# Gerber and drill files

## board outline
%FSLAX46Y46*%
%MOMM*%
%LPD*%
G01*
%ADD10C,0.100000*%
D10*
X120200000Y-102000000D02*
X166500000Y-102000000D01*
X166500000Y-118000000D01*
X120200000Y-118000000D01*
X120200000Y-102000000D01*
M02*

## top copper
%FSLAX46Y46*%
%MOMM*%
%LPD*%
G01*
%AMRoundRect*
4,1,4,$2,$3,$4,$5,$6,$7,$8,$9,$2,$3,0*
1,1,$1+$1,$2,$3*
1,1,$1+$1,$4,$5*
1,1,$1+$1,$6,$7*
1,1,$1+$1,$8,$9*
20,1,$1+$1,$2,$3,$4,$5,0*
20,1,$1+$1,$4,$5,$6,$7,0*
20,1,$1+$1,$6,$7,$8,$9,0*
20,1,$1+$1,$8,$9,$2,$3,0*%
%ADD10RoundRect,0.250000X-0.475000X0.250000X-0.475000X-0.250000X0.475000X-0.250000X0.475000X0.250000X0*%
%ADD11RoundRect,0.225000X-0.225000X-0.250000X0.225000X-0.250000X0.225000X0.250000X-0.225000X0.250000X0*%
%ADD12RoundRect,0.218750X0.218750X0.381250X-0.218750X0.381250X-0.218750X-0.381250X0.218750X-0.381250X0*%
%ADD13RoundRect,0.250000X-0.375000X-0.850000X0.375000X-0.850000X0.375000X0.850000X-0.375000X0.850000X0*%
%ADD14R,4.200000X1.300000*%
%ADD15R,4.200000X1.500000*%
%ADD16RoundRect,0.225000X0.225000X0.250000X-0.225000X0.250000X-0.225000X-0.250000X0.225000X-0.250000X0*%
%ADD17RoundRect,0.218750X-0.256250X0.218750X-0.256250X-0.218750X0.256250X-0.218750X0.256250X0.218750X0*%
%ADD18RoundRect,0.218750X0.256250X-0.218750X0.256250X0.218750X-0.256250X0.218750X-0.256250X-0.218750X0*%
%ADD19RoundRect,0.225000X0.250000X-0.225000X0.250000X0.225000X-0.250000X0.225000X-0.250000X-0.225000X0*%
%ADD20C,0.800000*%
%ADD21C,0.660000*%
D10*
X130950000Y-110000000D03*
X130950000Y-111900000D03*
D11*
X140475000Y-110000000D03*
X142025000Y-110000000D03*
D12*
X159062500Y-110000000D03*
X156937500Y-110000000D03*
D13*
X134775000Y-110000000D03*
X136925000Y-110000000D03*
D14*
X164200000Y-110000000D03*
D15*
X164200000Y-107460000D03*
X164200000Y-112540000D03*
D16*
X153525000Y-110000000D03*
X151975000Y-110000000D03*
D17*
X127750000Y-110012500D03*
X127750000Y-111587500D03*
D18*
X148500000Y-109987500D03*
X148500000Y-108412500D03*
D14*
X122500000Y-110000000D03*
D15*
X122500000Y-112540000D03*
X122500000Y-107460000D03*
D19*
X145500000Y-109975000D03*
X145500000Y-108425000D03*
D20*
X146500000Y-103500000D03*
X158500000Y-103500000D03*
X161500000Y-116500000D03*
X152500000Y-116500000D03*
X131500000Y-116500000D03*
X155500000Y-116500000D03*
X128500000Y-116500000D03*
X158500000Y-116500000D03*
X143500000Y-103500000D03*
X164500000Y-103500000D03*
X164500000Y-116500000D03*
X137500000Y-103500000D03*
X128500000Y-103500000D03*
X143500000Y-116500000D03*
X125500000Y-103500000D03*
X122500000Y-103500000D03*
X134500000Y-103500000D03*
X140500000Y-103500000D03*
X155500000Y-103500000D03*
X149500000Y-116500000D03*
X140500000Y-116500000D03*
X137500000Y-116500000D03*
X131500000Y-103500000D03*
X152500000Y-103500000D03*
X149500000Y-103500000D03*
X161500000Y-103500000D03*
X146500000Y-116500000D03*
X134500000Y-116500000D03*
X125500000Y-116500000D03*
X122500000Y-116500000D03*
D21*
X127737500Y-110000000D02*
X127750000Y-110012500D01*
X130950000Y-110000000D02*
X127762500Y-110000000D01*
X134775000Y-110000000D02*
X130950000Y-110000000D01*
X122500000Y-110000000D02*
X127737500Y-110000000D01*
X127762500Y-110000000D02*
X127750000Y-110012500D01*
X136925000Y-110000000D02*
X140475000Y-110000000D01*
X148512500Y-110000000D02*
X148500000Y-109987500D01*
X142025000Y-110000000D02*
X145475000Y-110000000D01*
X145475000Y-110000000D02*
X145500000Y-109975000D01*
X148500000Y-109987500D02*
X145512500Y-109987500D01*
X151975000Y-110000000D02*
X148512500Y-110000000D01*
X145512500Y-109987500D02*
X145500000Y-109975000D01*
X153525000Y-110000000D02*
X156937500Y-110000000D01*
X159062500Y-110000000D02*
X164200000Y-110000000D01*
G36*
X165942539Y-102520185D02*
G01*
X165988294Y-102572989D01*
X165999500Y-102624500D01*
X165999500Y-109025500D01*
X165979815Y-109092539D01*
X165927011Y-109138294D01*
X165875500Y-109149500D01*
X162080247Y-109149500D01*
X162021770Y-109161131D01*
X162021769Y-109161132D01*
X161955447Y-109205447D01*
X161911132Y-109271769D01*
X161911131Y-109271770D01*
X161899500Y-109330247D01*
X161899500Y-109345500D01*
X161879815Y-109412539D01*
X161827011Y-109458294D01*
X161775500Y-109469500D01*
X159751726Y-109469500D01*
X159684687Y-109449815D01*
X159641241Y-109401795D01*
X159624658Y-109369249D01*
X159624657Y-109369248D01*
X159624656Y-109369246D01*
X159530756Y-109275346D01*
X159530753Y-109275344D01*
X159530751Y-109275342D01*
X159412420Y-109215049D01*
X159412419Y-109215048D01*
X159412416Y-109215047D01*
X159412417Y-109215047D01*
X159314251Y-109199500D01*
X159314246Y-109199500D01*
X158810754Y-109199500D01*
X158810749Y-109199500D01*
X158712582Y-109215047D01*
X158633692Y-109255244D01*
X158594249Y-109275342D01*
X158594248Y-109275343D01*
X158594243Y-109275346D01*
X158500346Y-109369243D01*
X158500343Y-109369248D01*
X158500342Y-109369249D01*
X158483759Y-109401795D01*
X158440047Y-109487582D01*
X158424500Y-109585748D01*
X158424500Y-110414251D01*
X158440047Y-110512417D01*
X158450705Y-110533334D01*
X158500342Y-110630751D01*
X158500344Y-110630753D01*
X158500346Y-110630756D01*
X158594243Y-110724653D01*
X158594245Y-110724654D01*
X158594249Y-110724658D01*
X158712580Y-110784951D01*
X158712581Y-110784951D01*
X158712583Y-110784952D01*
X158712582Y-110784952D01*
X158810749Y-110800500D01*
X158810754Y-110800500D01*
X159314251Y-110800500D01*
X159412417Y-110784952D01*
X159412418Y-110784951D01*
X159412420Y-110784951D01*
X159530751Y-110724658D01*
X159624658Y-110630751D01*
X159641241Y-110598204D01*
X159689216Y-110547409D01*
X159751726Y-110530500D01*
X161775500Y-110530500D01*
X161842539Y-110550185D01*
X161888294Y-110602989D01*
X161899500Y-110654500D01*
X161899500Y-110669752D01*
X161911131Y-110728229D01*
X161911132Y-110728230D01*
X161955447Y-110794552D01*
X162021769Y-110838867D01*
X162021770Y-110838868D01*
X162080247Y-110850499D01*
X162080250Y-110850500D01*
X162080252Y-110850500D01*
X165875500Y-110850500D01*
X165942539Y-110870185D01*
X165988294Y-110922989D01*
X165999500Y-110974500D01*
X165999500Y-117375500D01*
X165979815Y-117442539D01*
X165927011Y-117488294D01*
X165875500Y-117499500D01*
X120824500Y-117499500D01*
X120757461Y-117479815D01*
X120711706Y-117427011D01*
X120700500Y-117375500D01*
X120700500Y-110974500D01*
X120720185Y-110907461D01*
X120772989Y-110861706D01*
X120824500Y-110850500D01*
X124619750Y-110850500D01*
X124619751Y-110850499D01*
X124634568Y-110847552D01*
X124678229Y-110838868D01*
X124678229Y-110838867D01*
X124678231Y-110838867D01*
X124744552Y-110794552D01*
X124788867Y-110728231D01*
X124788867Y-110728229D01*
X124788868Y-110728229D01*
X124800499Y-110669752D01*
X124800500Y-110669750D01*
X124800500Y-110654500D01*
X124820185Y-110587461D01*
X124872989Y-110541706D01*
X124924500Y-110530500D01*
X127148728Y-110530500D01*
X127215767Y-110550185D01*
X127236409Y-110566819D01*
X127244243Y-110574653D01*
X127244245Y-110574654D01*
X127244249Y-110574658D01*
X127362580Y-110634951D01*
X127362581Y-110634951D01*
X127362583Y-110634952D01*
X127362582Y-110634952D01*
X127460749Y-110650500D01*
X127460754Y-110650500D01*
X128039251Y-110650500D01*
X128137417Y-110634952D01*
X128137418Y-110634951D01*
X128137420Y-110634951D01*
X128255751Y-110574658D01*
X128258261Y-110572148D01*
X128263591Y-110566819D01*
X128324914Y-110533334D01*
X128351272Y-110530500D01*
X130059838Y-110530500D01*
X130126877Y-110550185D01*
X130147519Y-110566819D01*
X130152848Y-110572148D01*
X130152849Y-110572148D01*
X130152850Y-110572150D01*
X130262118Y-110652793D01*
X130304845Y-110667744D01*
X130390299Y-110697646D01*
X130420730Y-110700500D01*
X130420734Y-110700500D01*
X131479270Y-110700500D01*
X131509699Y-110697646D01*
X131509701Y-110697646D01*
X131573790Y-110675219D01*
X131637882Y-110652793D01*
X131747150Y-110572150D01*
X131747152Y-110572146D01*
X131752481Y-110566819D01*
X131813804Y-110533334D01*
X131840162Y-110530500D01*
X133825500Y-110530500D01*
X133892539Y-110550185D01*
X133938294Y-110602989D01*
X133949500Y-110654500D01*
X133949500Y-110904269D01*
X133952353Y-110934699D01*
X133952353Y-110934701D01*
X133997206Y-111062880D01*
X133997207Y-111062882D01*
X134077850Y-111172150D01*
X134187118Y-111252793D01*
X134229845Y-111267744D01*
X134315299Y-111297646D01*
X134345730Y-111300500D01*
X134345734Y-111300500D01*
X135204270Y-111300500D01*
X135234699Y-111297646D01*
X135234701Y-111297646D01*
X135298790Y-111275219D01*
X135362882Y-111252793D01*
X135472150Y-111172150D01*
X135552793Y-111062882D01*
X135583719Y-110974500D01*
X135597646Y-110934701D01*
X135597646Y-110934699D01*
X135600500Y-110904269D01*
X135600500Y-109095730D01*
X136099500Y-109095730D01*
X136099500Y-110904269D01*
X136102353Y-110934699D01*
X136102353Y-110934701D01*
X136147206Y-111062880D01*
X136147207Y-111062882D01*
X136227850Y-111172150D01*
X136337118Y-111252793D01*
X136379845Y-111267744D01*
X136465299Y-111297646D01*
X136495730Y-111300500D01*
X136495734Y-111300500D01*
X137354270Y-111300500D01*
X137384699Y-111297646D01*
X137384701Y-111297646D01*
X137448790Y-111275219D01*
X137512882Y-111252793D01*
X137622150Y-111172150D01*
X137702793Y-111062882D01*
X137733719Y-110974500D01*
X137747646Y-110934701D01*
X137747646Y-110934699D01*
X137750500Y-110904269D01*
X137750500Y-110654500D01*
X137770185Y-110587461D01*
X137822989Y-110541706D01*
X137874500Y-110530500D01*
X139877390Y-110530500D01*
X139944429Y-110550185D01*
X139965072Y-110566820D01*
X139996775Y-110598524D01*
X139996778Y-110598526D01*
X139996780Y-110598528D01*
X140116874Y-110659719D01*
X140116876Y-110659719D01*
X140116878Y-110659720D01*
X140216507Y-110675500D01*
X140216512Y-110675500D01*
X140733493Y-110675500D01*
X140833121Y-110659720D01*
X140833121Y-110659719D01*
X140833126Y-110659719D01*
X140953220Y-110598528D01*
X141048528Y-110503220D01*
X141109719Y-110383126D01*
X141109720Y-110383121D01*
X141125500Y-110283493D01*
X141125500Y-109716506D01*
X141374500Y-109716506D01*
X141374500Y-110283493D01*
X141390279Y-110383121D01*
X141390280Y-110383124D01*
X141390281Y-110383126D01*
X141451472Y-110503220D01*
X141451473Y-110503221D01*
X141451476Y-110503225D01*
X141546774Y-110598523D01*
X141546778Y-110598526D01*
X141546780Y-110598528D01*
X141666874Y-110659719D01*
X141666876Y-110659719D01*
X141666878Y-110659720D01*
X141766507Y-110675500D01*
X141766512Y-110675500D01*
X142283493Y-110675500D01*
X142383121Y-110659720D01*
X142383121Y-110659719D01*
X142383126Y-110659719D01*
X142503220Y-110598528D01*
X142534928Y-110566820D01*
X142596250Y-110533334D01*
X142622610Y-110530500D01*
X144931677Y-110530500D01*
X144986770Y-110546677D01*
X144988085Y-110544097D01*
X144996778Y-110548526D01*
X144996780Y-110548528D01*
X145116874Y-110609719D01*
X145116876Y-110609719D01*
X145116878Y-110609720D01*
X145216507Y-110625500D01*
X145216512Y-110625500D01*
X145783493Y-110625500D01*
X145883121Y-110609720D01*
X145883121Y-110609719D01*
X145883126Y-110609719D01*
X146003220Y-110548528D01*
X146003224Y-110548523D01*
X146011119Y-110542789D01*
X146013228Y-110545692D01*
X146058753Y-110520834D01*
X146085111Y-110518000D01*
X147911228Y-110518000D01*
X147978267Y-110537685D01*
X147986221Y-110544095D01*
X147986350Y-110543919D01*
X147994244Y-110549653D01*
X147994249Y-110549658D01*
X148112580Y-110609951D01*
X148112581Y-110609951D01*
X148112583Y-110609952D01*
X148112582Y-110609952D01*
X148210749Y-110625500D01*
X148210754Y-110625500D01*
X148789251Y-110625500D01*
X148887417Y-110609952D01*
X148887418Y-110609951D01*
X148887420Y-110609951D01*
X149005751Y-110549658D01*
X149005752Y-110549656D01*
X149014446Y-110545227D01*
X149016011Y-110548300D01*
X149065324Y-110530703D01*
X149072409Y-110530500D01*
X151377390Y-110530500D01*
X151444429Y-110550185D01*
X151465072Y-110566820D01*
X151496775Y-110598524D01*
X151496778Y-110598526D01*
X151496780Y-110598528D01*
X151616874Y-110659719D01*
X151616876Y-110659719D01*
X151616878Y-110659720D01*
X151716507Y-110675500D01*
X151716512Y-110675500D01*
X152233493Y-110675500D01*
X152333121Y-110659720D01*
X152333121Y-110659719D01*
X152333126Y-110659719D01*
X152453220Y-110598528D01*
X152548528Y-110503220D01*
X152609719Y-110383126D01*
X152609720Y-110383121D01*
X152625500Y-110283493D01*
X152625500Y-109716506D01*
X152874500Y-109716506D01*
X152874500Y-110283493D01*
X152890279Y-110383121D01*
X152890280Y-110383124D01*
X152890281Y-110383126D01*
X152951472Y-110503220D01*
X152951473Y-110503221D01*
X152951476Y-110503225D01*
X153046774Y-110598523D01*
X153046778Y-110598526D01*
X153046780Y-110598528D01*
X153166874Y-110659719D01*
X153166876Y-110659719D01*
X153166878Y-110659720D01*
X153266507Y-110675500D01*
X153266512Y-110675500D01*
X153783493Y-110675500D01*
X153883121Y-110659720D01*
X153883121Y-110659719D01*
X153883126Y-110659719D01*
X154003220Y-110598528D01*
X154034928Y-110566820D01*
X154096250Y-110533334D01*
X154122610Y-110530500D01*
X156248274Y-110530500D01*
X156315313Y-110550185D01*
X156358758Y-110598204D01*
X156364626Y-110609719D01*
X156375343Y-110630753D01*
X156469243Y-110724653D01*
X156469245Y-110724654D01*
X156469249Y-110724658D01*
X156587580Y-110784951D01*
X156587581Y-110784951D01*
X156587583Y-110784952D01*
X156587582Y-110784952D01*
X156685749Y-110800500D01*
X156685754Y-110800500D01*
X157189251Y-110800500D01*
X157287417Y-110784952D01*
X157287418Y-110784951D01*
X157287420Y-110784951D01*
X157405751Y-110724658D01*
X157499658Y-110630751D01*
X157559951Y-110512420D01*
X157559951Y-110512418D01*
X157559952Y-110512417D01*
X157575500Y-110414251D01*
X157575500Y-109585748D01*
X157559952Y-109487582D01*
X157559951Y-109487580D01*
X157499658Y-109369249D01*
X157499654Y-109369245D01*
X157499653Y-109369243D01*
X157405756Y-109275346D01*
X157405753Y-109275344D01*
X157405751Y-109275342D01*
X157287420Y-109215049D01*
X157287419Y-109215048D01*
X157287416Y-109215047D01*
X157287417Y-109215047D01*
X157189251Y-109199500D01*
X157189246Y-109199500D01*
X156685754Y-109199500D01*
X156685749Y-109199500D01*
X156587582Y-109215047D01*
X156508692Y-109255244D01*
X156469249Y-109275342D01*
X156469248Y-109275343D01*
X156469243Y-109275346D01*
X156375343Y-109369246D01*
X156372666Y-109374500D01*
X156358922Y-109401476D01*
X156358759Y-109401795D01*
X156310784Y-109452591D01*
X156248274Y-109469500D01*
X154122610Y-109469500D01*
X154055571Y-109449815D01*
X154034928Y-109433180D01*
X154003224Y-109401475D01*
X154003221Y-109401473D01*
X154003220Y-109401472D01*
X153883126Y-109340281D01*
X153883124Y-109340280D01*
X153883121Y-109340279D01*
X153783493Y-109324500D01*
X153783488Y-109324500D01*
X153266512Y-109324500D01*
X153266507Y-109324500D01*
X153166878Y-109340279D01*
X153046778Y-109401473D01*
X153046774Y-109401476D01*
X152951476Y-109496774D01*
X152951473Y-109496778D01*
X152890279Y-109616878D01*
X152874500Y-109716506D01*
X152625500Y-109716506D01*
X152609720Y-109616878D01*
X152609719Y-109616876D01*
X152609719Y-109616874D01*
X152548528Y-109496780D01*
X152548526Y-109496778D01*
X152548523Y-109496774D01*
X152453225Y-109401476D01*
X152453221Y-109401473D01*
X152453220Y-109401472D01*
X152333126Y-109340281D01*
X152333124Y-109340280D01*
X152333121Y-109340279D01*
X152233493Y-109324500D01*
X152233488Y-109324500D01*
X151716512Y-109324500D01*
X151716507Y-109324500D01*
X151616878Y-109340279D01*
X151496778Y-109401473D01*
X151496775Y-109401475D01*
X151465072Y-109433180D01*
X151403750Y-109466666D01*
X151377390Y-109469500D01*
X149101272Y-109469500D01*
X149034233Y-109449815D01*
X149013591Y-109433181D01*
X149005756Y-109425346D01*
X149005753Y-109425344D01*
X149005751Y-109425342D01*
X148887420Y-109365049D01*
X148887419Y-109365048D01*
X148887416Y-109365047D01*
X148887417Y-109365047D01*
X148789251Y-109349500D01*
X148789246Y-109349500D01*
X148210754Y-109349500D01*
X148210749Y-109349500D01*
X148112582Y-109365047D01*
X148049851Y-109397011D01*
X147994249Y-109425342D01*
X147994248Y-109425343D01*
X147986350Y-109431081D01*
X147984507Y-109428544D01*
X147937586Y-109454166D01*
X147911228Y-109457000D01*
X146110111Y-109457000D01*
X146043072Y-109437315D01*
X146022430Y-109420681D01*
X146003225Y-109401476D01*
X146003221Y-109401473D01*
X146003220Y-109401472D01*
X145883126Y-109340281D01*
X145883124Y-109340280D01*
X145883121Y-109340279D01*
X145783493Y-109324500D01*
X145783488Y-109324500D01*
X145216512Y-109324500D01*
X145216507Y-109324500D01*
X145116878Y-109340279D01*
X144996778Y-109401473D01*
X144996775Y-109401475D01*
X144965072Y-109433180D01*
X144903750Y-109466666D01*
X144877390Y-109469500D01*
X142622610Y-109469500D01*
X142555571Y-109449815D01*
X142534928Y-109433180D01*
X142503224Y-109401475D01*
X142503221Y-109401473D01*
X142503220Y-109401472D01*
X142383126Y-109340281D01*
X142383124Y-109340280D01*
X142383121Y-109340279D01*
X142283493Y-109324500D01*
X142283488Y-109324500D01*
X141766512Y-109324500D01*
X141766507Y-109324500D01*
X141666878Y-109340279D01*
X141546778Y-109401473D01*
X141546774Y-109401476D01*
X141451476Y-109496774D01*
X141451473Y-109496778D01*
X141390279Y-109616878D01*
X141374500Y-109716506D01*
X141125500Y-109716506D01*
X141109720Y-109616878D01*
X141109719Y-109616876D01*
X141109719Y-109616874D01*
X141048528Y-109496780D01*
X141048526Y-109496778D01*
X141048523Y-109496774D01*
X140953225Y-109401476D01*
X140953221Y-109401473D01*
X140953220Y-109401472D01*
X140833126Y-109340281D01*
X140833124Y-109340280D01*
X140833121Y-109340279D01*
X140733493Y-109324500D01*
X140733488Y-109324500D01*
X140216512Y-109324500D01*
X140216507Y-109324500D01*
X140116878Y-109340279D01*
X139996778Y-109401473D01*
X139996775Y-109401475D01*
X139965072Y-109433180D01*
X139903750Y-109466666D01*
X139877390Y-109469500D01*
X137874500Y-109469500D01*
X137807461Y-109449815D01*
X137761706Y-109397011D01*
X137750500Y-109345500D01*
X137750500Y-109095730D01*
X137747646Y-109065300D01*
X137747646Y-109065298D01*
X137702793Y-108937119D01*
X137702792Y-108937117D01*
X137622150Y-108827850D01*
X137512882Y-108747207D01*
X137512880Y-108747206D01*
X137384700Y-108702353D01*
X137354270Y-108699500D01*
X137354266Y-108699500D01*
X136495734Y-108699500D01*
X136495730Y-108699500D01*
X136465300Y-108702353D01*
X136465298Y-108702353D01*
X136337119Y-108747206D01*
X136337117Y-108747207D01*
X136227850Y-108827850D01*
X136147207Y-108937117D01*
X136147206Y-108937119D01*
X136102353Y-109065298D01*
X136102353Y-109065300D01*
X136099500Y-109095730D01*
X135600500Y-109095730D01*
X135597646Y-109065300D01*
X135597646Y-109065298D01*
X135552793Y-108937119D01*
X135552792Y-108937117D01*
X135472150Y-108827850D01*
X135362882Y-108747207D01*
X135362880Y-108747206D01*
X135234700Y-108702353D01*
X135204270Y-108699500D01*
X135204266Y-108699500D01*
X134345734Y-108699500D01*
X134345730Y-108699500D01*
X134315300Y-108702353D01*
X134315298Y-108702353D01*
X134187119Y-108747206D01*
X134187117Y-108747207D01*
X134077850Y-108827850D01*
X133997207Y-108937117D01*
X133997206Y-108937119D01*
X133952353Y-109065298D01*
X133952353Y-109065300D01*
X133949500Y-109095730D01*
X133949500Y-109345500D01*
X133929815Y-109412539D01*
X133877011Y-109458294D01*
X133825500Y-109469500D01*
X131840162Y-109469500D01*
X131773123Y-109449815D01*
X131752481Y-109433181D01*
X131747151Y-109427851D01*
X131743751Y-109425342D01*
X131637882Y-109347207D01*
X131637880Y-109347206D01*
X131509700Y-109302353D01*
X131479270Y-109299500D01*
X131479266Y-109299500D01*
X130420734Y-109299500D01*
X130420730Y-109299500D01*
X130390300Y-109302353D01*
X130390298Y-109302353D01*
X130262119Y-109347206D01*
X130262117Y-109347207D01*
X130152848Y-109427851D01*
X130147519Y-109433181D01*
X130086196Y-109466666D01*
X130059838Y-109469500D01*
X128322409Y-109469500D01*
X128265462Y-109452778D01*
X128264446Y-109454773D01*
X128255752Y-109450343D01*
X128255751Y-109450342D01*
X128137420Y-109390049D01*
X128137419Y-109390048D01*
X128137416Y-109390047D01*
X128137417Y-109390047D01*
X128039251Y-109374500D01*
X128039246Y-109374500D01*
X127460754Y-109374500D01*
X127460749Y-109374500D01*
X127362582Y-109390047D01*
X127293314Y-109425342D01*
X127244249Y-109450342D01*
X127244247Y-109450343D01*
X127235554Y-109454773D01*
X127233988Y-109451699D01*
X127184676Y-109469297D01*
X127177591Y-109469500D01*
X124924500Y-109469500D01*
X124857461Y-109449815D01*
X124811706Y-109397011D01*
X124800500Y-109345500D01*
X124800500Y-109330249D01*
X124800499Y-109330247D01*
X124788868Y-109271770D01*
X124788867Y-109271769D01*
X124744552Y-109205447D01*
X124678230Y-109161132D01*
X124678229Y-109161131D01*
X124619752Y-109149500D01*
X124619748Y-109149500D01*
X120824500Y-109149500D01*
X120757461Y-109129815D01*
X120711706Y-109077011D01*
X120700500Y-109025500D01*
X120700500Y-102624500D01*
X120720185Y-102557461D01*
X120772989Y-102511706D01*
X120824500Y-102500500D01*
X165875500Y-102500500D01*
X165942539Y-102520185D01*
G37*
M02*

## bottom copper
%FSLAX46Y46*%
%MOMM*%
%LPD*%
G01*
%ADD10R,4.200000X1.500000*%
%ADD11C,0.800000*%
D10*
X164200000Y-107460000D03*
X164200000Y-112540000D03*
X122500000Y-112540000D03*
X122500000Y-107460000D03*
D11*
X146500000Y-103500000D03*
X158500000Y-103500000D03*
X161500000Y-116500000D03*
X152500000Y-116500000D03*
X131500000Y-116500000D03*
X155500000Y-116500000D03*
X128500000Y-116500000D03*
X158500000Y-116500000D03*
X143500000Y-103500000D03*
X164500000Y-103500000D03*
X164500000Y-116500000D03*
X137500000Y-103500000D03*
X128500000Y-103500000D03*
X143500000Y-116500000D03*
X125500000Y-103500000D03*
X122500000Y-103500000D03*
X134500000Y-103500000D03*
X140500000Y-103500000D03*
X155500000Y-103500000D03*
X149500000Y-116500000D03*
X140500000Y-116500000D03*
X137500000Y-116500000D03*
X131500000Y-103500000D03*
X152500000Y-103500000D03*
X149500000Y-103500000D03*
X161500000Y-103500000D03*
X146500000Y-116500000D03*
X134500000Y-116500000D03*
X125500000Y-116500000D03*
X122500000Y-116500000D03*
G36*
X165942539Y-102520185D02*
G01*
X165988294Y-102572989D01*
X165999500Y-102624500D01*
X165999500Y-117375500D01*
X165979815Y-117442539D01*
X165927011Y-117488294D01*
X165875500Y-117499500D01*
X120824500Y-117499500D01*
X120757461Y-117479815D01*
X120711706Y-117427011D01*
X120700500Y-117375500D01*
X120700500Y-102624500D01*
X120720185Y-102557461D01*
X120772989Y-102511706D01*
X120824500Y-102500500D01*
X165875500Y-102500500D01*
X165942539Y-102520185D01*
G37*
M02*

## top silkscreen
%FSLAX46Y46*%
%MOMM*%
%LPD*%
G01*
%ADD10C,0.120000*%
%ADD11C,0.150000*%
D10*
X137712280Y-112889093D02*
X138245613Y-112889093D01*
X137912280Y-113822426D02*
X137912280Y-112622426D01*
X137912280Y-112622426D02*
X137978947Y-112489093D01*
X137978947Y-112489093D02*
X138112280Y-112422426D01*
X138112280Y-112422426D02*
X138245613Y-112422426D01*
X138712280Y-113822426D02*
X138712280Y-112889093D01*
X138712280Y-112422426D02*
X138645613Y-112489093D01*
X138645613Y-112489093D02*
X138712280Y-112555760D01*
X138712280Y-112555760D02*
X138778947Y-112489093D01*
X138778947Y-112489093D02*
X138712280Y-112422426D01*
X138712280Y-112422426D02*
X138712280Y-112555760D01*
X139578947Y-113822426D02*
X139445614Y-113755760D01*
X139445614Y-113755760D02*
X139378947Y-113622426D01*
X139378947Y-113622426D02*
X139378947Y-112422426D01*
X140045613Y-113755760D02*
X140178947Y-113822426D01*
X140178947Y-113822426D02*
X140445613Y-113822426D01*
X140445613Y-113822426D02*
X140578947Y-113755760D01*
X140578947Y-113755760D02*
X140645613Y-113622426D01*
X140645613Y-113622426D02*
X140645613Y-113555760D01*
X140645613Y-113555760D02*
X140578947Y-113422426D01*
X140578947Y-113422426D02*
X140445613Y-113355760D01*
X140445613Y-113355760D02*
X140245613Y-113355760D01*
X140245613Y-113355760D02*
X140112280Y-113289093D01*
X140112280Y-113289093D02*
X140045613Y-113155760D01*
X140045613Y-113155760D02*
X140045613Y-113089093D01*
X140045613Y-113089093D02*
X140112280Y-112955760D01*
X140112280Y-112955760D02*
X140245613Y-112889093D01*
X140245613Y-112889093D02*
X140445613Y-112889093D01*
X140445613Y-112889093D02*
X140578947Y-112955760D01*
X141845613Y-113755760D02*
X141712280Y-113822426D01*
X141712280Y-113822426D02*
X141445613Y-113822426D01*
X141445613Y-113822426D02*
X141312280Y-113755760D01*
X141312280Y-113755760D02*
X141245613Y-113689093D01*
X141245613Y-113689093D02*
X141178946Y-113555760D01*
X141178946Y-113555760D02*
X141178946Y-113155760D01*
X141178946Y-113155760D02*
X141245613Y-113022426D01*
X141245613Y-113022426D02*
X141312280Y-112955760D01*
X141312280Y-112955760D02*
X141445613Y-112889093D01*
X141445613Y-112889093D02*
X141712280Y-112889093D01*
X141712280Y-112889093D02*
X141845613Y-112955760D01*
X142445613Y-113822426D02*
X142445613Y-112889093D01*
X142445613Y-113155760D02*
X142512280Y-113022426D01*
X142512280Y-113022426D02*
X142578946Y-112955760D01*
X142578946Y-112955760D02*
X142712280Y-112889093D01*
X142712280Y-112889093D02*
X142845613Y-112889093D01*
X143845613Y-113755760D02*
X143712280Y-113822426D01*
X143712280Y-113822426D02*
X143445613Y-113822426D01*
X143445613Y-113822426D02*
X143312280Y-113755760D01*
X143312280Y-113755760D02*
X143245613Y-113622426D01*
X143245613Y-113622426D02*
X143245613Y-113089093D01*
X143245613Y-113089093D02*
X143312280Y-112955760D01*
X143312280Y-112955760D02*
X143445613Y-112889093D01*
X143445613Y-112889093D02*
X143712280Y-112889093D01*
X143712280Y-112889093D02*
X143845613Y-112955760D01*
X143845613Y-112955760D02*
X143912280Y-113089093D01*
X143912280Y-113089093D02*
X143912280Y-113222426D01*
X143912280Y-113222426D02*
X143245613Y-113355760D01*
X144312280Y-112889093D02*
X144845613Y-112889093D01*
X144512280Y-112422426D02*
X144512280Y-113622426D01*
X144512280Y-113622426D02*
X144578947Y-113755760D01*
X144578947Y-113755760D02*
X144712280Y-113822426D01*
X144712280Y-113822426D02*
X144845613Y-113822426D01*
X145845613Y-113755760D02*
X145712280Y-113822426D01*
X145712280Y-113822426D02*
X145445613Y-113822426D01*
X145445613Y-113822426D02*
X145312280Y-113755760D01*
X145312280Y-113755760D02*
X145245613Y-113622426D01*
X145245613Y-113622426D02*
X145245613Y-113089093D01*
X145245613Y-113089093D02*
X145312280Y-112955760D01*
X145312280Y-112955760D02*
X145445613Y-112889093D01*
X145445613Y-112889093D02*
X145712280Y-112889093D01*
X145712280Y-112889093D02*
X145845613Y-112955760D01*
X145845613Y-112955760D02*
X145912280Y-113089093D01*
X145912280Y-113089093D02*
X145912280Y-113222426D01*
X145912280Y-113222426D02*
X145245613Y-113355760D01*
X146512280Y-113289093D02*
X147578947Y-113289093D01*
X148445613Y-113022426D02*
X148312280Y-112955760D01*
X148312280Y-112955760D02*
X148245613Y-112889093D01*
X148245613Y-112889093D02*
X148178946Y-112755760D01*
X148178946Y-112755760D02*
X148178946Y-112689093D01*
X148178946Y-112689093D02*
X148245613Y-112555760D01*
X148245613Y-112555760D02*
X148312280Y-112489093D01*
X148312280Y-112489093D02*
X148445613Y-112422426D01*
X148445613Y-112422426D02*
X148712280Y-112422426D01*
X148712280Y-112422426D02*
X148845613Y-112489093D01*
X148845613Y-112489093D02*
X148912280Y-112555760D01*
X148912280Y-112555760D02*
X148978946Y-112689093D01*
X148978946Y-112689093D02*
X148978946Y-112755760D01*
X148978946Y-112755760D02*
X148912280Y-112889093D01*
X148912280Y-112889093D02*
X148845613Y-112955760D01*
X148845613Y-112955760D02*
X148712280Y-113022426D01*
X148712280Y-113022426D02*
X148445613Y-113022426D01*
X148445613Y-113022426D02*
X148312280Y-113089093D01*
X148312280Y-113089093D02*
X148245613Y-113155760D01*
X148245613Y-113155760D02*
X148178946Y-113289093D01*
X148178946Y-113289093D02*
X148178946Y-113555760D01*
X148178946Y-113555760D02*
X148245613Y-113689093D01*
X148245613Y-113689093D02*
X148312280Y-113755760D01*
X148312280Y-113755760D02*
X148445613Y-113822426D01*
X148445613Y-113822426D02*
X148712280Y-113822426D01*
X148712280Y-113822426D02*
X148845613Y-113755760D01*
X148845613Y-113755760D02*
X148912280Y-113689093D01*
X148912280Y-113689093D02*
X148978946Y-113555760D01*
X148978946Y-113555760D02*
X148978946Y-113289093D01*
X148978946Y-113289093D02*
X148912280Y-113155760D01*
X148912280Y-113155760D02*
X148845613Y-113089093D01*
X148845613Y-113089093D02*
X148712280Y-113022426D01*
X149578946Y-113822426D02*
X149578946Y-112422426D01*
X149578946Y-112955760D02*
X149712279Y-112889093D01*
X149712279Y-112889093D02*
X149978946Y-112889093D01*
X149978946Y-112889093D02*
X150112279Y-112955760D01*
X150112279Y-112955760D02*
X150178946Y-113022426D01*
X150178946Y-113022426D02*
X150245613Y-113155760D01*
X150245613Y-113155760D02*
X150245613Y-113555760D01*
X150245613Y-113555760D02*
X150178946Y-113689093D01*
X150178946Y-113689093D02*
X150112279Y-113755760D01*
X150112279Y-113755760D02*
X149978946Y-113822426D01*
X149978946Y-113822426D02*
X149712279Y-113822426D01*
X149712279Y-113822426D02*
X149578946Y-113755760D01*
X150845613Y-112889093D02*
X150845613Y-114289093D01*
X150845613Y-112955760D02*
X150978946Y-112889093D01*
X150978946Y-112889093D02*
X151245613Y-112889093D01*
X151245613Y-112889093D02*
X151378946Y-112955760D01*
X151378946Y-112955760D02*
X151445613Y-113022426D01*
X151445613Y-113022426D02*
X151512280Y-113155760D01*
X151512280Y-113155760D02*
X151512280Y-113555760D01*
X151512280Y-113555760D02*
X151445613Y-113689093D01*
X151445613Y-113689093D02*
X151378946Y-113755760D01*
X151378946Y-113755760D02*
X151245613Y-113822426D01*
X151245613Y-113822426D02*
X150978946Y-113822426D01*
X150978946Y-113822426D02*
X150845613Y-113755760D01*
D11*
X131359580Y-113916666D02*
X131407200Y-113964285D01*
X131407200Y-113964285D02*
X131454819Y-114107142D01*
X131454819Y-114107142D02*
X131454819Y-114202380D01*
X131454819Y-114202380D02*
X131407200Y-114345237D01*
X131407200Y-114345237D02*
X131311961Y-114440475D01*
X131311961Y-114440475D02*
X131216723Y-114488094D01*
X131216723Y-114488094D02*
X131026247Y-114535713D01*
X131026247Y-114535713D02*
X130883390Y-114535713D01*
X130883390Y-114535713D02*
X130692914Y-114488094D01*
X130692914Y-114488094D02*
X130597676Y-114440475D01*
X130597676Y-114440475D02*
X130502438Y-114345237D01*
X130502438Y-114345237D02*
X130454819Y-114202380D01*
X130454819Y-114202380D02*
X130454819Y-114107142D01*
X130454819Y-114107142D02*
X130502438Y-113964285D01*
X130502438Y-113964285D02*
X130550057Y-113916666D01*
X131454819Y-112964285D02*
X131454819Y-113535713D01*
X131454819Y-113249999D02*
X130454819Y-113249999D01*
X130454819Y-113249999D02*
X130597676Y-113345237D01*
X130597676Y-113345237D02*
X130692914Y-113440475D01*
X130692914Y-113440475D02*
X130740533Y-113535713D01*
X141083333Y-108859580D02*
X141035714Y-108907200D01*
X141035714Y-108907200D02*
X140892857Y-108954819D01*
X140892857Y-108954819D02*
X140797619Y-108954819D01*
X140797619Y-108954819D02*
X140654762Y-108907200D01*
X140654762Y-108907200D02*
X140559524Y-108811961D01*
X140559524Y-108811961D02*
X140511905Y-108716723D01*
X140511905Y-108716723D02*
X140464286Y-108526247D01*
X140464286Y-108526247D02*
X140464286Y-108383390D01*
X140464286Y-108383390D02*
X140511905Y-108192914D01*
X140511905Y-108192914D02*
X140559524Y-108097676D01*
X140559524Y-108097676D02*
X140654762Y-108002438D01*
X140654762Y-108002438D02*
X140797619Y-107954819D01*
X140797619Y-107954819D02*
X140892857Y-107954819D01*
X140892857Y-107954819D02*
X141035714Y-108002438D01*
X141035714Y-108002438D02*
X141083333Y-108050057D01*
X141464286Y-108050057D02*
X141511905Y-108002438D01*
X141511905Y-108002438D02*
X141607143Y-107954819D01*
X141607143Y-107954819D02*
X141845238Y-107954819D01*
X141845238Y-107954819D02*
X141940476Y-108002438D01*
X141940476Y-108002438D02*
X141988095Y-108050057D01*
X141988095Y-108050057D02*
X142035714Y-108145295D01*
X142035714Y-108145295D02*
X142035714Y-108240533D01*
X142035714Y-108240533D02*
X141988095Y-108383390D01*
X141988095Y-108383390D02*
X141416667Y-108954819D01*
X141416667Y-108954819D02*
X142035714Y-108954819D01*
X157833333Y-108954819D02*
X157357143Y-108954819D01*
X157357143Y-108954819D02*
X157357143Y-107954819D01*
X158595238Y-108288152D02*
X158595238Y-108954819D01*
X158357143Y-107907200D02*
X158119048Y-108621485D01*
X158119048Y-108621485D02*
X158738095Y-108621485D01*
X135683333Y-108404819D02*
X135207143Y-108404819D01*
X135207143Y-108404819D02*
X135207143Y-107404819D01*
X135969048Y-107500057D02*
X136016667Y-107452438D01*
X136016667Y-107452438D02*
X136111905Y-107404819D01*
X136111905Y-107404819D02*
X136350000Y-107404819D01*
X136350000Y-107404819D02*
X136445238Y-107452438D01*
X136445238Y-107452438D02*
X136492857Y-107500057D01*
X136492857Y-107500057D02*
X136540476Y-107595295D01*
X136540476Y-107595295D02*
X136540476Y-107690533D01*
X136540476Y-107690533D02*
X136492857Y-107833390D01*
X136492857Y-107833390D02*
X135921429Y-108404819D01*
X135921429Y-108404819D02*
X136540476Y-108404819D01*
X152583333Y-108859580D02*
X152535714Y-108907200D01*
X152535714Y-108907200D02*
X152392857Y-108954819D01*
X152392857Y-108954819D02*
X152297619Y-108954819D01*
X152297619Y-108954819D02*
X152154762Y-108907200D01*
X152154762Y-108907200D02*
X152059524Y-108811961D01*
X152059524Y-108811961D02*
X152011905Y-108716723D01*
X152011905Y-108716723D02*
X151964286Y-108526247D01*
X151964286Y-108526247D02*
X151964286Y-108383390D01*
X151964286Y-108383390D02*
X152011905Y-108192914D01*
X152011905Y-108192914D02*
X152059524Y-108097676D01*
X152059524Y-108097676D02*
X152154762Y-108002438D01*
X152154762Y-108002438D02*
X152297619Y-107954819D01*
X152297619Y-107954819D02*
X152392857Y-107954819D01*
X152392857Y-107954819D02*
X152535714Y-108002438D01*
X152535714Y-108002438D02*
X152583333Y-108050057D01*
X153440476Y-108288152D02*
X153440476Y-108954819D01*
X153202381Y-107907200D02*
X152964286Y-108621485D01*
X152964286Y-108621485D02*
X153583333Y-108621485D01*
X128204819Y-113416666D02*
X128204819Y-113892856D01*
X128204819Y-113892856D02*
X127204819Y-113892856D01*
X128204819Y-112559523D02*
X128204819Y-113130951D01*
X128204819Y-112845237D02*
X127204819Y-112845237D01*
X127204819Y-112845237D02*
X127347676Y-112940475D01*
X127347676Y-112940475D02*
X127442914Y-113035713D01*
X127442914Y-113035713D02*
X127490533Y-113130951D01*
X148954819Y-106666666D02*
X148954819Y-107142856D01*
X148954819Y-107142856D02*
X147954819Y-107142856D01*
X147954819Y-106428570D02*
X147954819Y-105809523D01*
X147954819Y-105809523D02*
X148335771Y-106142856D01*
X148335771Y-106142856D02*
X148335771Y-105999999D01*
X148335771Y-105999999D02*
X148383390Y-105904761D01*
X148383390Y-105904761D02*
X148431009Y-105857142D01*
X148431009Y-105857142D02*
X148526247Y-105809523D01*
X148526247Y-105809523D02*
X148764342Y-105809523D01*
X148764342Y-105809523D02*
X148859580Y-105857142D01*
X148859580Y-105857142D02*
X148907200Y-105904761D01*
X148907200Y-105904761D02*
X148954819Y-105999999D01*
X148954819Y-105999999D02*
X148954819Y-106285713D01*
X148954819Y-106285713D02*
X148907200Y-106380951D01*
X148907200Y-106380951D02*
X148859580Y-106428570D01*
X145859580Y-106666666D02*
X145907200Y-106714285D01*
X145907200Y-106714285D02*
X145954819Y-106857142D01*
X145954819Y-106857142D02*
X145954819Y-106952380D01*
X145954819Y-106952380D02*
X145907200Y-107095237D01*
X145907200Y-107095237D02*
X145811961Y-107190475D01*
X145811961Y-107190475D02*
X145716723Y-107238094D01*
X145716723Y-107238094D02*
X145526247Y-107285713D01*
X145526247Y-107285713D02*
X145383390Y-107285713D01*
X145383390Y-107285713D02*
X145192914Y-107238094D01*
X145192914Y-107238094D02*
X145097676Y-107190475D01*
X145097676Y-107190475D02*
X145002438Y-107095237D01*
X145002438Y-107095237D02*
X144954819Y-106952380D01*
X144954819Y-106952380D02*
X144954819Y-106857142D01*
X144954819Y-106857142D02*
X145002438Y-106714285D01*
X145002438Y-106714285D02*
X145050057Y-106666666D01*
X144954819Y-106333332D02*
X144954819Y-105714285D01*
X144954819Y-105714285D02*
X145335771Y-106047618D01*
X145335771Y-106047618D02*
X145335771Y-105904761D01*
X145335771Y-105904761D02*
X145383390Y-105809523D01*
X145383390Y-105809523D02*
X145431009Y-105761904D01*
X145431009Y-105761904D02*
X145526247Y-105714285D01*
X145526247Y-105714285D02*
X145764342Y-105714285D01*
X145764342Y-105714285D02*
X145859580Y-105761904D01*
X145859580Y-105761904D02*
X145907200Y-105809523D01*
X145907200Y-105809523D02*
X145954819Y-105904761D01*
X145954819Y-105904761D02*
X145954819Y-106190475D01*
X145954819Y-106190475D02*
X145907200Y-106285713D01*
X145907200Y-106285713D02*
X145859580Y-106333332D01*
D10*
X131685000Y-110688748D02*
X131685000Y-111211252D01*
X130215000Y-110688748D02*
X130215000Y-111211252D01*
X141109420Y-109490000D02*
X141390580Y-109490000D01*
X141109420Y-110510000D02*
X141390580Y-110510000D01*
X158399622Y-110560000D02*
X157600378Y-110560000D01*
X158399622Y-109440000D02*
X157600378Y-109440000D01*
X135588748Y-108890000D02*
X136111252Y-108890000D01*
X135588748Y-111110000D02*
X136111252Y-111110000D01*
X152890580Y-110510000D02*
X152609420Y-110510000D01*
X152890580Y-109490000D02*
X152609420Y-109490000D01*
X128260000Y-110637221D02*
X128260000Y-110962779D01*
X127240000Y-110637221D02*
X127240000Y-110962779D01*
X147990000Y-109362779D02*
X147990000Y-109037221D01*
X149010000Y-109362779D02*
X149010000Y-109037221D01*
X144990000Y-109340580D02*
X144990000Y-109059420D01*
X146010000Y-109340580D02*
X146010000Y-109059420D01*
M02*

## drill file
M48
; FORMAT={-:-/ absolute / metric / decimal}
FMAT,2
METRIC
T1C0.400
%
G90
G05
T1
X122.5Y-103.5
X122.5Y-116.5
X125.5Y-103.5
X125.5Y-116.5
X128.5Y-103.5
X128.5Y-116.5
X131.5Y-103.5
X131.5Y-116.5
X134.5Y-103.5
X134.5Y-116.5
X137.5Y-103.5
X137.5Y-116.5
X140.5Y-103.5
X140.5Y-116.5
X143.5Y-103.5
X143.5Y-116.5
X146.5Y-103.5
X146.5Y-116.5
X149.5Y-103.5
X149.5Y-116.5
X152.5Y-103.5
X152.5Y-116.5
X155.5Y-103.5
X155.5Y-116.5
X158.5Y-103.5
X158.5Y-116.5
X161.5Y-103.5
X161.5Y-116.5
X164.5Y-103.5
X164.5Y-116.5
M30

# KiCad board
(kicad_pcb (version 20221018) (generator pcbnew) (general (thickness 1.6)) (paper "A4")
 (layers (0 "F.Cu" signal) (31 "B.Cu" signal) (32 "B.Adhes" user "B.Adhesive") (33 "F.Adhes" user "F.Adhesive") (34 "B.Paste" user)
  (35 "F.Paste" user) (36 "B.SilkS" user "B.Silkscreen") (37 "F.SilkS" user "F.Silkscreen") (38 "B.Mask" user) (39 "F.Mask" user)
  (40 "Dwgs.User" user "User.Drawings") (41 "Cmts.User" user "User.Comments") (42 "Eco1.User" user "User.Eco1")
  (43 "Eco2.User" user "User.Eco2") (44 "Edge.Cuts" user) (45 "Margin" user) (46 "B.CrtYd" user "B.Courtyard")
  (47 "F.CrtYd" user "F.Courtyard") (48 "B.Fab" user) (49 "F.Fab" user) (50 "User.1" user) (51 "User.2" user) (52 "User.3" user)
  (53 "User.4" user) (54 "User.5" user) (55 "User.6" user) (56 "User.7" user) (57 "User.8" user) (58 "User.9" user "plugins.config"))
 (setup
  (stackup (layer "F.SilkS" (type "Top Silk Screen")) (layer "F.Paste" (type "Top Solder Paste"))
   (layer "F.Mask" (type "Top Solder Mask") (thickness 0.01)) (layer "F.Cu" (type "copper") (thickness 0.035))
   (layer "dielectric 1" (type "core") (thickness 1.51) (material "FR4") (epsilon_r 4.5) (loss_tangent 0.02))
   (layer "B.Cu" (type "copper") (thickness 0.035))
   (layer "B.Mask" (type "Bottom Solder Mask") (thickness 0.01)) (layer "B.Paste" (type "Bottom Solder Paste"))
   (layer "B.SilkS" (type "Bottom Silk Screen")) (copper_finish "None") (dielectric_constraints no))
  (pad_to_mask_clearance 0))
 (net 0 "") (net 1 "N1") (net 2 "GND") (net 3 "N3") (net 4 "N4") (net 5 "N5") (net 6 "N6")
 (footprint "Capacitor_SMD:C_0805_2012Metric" (layer "F.Cu") (at 130.95 110.95 -90)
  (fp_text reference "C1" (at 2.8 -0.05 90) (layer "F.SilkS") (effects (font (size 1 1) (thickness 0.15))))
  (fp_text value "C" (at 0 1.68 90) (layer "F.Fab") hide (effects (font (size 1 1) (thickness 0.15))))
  (fp_line (start -0.261252 -0.735) (end 0.261252 -0.735) (stroke (width 0.12) (type solid)) (layer "F.SilkS"))
  (fp_line (start -0.261252 0.735) (end 0.261252 0.735) (stroke (width 0.12) (type solid)) (layer "F.SilkS"))
  (pad "1" smd roundrect (at -0.95 0 270) (size 1 1.45) (layers "F.Cu" "F.Paste" "F.Mask") (roundrect_rratio 0.25) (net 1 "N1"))
  (pad "2" smd roundrect (at 0.95 0 270) (size 1 1.45) (layers "F.Cu" "F.Paste" "F.Mask") (roundrect_rratio 0.25) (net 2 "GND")))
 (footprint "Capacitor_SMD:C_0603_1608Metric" (layer "F.Cu") (at 141.25 110)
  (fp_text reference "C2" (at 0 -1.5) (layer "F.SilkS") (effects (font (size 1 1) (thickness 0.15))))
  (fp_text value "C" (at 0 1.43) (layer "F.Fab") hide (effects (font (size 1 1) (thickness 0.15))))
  (fp_line (start -0.14058 -0.51) (end 0.14058 -0.51) (stroke (width 0.12) (type solid)) (layer "F.SilkS"))
  (fp_line (start -0.14058 0.51) (end 0.14058 0.51) (stroke (width 0.12) (type solid)) (layer "F.SilkS"))
  (pad "1" smd roundrect (at -0.775 0) (size 0.9 0.95) (layers "F.Cu" "F.Paste" "F.Mask") (roundrect_rratio 0.25) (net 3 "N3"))
  (pad "2" smd roundrect (at 0.775 0) (size 0.9 0.95) (layers "F.Cu" "F.Paste" "F.Mask") (roundrect_rratio 0.25) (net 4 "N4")))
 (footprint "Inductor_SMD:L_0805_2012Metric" (layer "F.Cu") (at 158 110 180)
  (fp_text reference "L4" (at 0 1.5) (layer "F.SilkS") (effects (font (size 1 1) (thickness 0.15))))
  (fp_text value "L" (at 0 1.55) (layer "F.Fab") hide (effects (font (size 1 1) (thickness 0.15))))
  (fp_line (start -0.399622 -0.56) (end 0.399622 -0.56) (stroke (width 0.12) (type solid)) (layer "F.SilkS"))
  (fp_line (start -0.399622 0.56) (end 0.399622 0.56) (stroke (width 0.12) (type solid)) (layer "F.SilkS"))
  (pad "1" smd roundrect (at -1.0625 0 180) (size 0.875 1.2) (layers "F.Cu" "F.Paste" "F.Mask") (roundrect_rratio 0.25) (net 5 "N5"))
  (pad "2" smd roundrect (at 1.0625 0 180) (size 0.875 1.2) (layers "F.Cu" "F.Paste" "F.Mask") (roundrect_rratio 0.25) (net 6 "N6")))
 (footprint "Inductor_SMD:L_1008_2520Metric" (layer "F.Cu") (at 135.85 110)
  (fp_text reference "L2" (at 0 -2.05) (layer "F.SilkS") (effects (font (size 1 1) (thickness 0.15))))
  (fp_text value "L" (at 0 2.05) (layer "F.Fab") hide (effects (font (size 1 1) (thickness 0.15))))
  (fp_line (start -0.261252 -1.11) (end 0.261252 -1.11) (stroke (width 0.12) (type solid)) (layer "F.SilkS"))
  (fp_line (start -0.261252 1.11) (end 0.261252 1.11) (stroke (width 0.12) (type solid)) (layer "F.SilkS"))
  (pad "1" smd roundrect (at -1.075 0) (size 1.25 2.2) (layers "F.Cu" "F.Paste" "F.Mask") (roundrect_rratio 0.2) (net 1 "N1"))
  (pad "2" smd roundrect (at 1.075 0) (size 1.25 2.2) (layers "F.Cu" "F.Paste" "F.Mask") (roundrect_rratio 0.2) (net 3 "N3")))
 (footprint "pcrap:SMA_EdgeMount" (layer "F.Cu") (at 163.2 110 -90)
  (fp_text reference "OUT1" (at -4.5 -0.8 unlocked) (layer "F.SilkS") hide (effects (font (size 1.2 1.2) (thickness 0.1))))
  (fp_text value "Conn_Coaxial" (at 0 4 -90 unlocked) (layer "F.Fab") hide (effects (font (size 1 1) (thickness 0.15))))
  (pad "1" smd rect (at 0 -1 90) (size 1.3 4.2) (layers "F.Cu" "F.Paste" "F.Mask") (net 5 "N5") (thermal_bridge_angle 45))
  (pad "2" smd rect (at -2.54 -1 90) (size 1.5 4.2) (layers "F.Cu" "F.Paste" "F.Mask") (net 2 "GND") (thermal_bridge_angle 45))
  (pad "2" smd rect (at -2.54 -1 270) (size 1.5 4.2) (layers "B.Cu" "B.Paste" "B.Mask") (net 2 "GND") (thermal_bridge_angle 45))
  (pad "2" smd rect (at 2.54 -1 90) (size 1.5 4.2) (layers "F.Cu" "F.Paste" "F.Mask") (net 2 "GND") (thermal_bridge_angle 45))
  (pad "2" smd rect (at 2.54 -1 90) (size 1.5 4.2) (layers "B.Cu" "B.Paste" "B.Mask") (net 2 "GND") (thermal_bridge_angle 45)))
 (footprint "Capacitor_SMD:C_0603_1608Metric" (layer "F.Cu") (at 152.75 110 180)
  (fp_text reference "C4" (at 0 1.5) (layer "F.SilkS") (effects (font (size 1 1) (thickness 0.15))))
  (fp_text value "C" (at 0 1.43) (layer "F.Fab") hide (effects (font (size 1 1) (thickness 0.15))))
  (fp_line (start -0.14058 -0.51) (end 0.14058 -0.51) (stroke (width 0.12) (type solid)) (layer "F.SilkS"))
  (fp_line (start -0.14058 0.51) (end 0.14058 0.51) (stroke (width 0.12) (type solid)) (layer "F.SilkS"))
  (pad "1" smd roundrect (at -0.775 0 180) (size 0.9 0.95) (layers "F.Cu" "F.Paste" "F.Mask") (roundrect_rratio 0.25) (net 6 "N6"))
  (pad "2" smd roundrect (at 0.775 0 180) (size 0.9 0.95) (layers "F.Cu" "F.Paste" "F.Mask") (roundrect_rratio 0.25) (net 4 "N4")))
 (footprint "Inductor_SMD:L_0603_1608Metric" (layer "F.Cu") (at 127.75 110.8 -90)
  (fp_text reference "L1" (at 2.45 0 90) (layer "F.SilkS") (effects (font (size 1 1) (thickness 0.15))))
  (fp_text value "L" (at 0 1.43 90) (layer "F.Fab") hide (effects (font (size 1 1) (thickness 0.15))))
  (fp_line (start -0.162779 -0.51) (end 0.162779 -0.51) (stroke (width 0.12) (type solid)) (layer "F.SilkS"))
  (fp_line (start -0.162779 0.51) (end 0.162779 0.51) (stroke (width 0.12) (type solid)) (layer "F.SilkS"))
  (pad "1" smd roundrect (at -0.7875 0 270) (size 0.875 0.95) (layers "F.Cu" "F.Paste" "F.Mask") (roundrect_rratio 0.25) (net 1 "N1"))
  (pad "2" smd roundrect (at 0.7875 0 270) (size 0.875 0.95) (layers "F.Cu" "F.Paste" "F.Mask") (roundrect_rratio 0.25) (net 2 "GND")))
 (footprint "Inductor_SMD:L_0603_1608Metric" (layer "F.Cu") (at 148.5 109.2 90)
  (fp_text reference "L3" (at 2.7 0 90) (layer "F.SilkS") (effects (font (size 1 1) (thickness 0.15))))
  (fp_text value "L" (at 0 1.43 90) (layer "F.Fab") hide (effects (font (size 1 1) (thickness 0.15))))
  (fp_line (start -0.162779 -0.51) (end 0.162779 -0.51) (stroke (width 0.12) (type solid)) (layer "F.SilkS"))
  (fp_line (start -0.162779 0.51) (end 0.162779 0.51) (stroke (width 0.12) (type solid)) (layer "F.SilkS"))
  (pad "1" smd roundrect (at -0.7875 0 90) (size 0.875 0.95) (layers "F.Cu" "F.Paste" "F.Mask") (roundrect_rratio 0.25) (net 4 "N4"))
  (pad "2" smd roundrect (at 0.7875 0 90) (size 0.875 0.95) (layers "F.Cu" "F.Paste" "F.Mask") (roundrect_rratio 0.25) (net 2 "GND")))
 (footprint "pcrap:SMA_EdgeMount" (layer "F.Cu") (at 123.5 110 90)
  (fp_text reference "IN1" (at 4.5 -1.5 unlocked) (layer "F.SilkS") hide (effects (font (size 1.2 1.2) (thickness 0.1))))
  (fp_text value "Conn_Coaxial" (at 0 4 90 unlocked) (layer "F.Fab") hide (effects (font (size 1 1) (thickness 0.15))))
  (pad "1" smd rect (at 0 -1 270) (size 1.3 4.2) (layers "F.Cu" "F.Paste" "F.Mask") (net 1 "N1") (thermal_bridge_angle 45))
  (pad "2" smd rect (at -2.54 -1 270) (size 1.5 4.2) (layers "F.Cu" "F.Paste" "F.Mask") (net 2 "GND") (thermal_bridge_angle 45))
  (pad "2" smd rect (at -2.54 -1 90) (size 1.5 4.2) (layers "B.Cu" "B.Paste" "B.Mask") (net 2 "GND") (thermal_bridge_angle 45))
  (pad "2" smd rect (at 2.54 -1 270) (size 1.5 4.2) (layers "F.Cu" "F.Paste" "F.Mask") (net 2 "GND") (thermal_bridge_angle 45))
  (pad "2" smd rect (at 2.54 -1 270) (size 1.5 4.2) (layers "B.Cu" "B.Paste" "B.Mask") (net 2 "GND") (thermal_bridge_angle 45)))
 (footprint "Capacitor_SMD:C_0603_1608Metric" (layer "F.Cu") (at 145.5 109.2 90)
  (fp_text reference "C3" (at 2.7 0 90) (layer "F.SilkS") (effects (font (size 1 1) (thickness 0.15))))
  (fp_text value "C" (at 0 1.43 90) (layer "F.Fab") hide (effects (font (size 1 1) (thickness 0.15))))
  (fp_line (start -0.14058 -0.51) (end 0.14058 -0.51) (stroke (width 0.12) (type solid)) (layer "F.SilkS"))
  (fp_line (start -0.14058 0.51) (end 0.14058 0.51) (stroke (width 0.12) (type solid)) (layer "F.SilkS"))
  (pad "1" smd roundrect (at -0.775 0 90) (size 0.9 0.95) (layers "F.Cu" "F.Paste" "F.Mask") (roundrect_rratio 0.25) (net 4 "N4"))
  (pad "2" smd roundrect (at 0.775 0 90) (size 0.9 0.95) (layers "F.Cu" "F.Paste" "F.Mask") (roundrect_rratio 0.25) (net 2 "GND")))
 (gr_rect (start 120.2 102) (end 166.5 118) (stroke (width 0.1) (type default)) (fill none) (layer "Edge.Cuts"))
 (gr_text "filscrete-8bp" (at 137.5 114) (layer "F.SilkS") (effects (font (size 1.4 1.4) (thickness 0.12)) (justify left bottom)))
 (segment (start 127.7375 110) (end 127.75 110.0125) (width 0.66) (layer "F.Cu") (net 1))
 (segment (start 130.95 110) (end 127.7625 110) (width 0.66) (layer "F.Cu") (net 1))
 (segment (start 134.775 110) (end 130.95 110) (width 0.66) (layer "F.Cu") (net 1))
 (segment (start 122.5 110) (end 127.7375 110) (width 0.66) (layer "F.Cu") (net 1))
 (segment (start 127.7625 110) (end 127.75 110.0125) (width 0.66) (layer "F.Cu") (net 1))
 (via (at 146.5 103.5) (size 0.8) (drill 0.4) (layers "F.Cu" "B.Cu") (free) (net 2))
 (via (at 158.5 103.5) (size 0.8) (drill 0.4) (layers "F.Cu" "B.Cu") (free) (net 2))
 (via (at 161.5 116.5) (size 0.8) (drill 0.4) (layers "F.Cu" "B.Cu") (free) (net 2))
 (via (at 152.5 116.5) (size 0.8) (drill 0.4) (layers "F.Cu" "B.Cu") (free) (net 2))
 (via (at 131.5 116.5) (size 0.8) (drill 0.4) (layers "F.Cu" "B.Cu") (free) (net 2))
 (via (at 155.5 116.5) (size 0.8) (drill 0.4) (layers "F.Cu" "B.Cu") (free) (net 2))
 (via (at 128.5 116.5) (size 0.8) (drill 0.4) (layers "F.Cu" "B.Cu") (free) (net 2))
 (via (at 158.5 116.5) (size 0.8) (drill 0.4) (layers "F.Cu" "B.Cu") (free) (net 2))
 (via (at 143.5 103.5) (size 0.8) (drill 0.4) (layers "F.Cu" "B.Cu") (free) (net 2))
 (via (at 164.5 103.5) (size 0.8) (drill 0.4) (layers "F.Cu" "B.Cu") (free) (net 2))
 (via (at 164.5 116.5) (size 0.8) (drill 0.4) (layers "F.Cu" "B.Cu") (free) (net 2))
 (via (at 137.5 103.5) (size 0.8) (drill 0.4) (layers "F.Cu" "B.Cu") (free) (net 2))
 (via (at 128.5 103.5) (size 0.8) (drill 0.4) (layers "F.Cu" "B.Cu") (free) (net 2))
 (via (at 143.5 116.5) (size 0.8) (drill 0.4) (layers "F.Cu" "B.Cu") (free) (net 2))
 (via (at 125.5 103.5) (size 0.8) (drill 0.4) (layers "F.Cu" "B.Cu") (free) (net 2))
 (via (at 122.5 103.5) (size 0.8) (drill 0.4) (layers "F.Cu" "B.Cu") (free) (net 2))
 (via (at 134.5 103.5) (size 0.8) (drill 0.4) (layers "F.Cu" "B.Cu") (free) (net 2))
 (via (at 140.5 103.5) (size 0.8) (drill 0.4) (layers "F.Cu" "B.Cu") (free) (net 2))
 (via (at 155.5 103.5) (size 0.8) (drill 0.4) (layers "F.Cu" "B.Cu") (free) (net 2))
 (via (at 149.5 116.5) (size 0.8) (drill 0.4) (layers "F.Cu" "B.Cu") (free) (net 2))
 (via (at 140.5 116.5) (size 0.8) (drill 0.4) (layers "F.Cu" "B.Cu") (free) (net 2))
 (via (at 137.5 116.5) (size 0.8) (drill 0.4) (layers "F.Cu" "B.Cu") (free) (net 2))
 (via (at 131.5 103.5) (size 0.8) (drill 0.4) (layers "F.Cu" "B.Cu") (free) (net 2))
 (via (at 152.5 103.5) (size 0.8) (drill 0.4) (layers "F.Cu" "B.Cu") (free) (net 2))
 (via (at 149.5 103.5) (size 0.8) (drill 0.4) (layers "F.Cu" "B.Cu") (free) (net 2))
 (via (at 161.5 103.5) (size 0.8) (drill 0.4) (layers "F.Cu" "B.Cu") (free) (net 2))
 (via (at 146.5 116.5) (size 0.8) (drill 0.4) (layers "F.Cu" "B.Cu") (free) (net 2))
 (via (at 134.5 116.5) (size 0.8) (drill 0.4) (layers "F.Cu" "B.Cu") (free) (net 2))
 (via (at 125.5 116.5) (size 0.8) (drill 0.4) (layers "F.Cu" "B.Cu") (free) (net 2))
 (via (at 122.5 116.5) (size 0.8) (drill 0.4) (layers "F.Cu" "B.Cu") (free) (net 2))
 (segment (start 136.925 110) (end 140.475 110) (width 0.66) (layer "F.Cu") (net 3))
 (segment (start 148.5125 110) (end 148.5 109.9875) (width 0.66) (layer "F.Cu") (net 4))
 (segment (start 142.025 110) (end 145.475 110) (width 0.66) (layer "F.Cu") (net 4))
 (segment (start 145.475 110) (end 145.5 109.975) (width 0.66) (layer "F.Cu") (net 4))
 (segment (start 148.5 109.9875) (end 145.5125 109.9875) (width 0.66) (layer "F.Cu") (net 4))
 (segment (start 151.975 110) (end 148.5125 110) (width 0.66) (layer "F.Cu") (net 4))
 (segment (start 145.5125 109.9875) (end 145.5 109.975) (width 0.66) (layer "F.Cu") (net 4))
 (segment (start 153.525 110) (end 156.9375 110) (width 0.66) (layer "F.Cu") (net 6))
 (segment (start 159.0625 110) (end 164.2 110) (width 0.66) (layer "F.Cu") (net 5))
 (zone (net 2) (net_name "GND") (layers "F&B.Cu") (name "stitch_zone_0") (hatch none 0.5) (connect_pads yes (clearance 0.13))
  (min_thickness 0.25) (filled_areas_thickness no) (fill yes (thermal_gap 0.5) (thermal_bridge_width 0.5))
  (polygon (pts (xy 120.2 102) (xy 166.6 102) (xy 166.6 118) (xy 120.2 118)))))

